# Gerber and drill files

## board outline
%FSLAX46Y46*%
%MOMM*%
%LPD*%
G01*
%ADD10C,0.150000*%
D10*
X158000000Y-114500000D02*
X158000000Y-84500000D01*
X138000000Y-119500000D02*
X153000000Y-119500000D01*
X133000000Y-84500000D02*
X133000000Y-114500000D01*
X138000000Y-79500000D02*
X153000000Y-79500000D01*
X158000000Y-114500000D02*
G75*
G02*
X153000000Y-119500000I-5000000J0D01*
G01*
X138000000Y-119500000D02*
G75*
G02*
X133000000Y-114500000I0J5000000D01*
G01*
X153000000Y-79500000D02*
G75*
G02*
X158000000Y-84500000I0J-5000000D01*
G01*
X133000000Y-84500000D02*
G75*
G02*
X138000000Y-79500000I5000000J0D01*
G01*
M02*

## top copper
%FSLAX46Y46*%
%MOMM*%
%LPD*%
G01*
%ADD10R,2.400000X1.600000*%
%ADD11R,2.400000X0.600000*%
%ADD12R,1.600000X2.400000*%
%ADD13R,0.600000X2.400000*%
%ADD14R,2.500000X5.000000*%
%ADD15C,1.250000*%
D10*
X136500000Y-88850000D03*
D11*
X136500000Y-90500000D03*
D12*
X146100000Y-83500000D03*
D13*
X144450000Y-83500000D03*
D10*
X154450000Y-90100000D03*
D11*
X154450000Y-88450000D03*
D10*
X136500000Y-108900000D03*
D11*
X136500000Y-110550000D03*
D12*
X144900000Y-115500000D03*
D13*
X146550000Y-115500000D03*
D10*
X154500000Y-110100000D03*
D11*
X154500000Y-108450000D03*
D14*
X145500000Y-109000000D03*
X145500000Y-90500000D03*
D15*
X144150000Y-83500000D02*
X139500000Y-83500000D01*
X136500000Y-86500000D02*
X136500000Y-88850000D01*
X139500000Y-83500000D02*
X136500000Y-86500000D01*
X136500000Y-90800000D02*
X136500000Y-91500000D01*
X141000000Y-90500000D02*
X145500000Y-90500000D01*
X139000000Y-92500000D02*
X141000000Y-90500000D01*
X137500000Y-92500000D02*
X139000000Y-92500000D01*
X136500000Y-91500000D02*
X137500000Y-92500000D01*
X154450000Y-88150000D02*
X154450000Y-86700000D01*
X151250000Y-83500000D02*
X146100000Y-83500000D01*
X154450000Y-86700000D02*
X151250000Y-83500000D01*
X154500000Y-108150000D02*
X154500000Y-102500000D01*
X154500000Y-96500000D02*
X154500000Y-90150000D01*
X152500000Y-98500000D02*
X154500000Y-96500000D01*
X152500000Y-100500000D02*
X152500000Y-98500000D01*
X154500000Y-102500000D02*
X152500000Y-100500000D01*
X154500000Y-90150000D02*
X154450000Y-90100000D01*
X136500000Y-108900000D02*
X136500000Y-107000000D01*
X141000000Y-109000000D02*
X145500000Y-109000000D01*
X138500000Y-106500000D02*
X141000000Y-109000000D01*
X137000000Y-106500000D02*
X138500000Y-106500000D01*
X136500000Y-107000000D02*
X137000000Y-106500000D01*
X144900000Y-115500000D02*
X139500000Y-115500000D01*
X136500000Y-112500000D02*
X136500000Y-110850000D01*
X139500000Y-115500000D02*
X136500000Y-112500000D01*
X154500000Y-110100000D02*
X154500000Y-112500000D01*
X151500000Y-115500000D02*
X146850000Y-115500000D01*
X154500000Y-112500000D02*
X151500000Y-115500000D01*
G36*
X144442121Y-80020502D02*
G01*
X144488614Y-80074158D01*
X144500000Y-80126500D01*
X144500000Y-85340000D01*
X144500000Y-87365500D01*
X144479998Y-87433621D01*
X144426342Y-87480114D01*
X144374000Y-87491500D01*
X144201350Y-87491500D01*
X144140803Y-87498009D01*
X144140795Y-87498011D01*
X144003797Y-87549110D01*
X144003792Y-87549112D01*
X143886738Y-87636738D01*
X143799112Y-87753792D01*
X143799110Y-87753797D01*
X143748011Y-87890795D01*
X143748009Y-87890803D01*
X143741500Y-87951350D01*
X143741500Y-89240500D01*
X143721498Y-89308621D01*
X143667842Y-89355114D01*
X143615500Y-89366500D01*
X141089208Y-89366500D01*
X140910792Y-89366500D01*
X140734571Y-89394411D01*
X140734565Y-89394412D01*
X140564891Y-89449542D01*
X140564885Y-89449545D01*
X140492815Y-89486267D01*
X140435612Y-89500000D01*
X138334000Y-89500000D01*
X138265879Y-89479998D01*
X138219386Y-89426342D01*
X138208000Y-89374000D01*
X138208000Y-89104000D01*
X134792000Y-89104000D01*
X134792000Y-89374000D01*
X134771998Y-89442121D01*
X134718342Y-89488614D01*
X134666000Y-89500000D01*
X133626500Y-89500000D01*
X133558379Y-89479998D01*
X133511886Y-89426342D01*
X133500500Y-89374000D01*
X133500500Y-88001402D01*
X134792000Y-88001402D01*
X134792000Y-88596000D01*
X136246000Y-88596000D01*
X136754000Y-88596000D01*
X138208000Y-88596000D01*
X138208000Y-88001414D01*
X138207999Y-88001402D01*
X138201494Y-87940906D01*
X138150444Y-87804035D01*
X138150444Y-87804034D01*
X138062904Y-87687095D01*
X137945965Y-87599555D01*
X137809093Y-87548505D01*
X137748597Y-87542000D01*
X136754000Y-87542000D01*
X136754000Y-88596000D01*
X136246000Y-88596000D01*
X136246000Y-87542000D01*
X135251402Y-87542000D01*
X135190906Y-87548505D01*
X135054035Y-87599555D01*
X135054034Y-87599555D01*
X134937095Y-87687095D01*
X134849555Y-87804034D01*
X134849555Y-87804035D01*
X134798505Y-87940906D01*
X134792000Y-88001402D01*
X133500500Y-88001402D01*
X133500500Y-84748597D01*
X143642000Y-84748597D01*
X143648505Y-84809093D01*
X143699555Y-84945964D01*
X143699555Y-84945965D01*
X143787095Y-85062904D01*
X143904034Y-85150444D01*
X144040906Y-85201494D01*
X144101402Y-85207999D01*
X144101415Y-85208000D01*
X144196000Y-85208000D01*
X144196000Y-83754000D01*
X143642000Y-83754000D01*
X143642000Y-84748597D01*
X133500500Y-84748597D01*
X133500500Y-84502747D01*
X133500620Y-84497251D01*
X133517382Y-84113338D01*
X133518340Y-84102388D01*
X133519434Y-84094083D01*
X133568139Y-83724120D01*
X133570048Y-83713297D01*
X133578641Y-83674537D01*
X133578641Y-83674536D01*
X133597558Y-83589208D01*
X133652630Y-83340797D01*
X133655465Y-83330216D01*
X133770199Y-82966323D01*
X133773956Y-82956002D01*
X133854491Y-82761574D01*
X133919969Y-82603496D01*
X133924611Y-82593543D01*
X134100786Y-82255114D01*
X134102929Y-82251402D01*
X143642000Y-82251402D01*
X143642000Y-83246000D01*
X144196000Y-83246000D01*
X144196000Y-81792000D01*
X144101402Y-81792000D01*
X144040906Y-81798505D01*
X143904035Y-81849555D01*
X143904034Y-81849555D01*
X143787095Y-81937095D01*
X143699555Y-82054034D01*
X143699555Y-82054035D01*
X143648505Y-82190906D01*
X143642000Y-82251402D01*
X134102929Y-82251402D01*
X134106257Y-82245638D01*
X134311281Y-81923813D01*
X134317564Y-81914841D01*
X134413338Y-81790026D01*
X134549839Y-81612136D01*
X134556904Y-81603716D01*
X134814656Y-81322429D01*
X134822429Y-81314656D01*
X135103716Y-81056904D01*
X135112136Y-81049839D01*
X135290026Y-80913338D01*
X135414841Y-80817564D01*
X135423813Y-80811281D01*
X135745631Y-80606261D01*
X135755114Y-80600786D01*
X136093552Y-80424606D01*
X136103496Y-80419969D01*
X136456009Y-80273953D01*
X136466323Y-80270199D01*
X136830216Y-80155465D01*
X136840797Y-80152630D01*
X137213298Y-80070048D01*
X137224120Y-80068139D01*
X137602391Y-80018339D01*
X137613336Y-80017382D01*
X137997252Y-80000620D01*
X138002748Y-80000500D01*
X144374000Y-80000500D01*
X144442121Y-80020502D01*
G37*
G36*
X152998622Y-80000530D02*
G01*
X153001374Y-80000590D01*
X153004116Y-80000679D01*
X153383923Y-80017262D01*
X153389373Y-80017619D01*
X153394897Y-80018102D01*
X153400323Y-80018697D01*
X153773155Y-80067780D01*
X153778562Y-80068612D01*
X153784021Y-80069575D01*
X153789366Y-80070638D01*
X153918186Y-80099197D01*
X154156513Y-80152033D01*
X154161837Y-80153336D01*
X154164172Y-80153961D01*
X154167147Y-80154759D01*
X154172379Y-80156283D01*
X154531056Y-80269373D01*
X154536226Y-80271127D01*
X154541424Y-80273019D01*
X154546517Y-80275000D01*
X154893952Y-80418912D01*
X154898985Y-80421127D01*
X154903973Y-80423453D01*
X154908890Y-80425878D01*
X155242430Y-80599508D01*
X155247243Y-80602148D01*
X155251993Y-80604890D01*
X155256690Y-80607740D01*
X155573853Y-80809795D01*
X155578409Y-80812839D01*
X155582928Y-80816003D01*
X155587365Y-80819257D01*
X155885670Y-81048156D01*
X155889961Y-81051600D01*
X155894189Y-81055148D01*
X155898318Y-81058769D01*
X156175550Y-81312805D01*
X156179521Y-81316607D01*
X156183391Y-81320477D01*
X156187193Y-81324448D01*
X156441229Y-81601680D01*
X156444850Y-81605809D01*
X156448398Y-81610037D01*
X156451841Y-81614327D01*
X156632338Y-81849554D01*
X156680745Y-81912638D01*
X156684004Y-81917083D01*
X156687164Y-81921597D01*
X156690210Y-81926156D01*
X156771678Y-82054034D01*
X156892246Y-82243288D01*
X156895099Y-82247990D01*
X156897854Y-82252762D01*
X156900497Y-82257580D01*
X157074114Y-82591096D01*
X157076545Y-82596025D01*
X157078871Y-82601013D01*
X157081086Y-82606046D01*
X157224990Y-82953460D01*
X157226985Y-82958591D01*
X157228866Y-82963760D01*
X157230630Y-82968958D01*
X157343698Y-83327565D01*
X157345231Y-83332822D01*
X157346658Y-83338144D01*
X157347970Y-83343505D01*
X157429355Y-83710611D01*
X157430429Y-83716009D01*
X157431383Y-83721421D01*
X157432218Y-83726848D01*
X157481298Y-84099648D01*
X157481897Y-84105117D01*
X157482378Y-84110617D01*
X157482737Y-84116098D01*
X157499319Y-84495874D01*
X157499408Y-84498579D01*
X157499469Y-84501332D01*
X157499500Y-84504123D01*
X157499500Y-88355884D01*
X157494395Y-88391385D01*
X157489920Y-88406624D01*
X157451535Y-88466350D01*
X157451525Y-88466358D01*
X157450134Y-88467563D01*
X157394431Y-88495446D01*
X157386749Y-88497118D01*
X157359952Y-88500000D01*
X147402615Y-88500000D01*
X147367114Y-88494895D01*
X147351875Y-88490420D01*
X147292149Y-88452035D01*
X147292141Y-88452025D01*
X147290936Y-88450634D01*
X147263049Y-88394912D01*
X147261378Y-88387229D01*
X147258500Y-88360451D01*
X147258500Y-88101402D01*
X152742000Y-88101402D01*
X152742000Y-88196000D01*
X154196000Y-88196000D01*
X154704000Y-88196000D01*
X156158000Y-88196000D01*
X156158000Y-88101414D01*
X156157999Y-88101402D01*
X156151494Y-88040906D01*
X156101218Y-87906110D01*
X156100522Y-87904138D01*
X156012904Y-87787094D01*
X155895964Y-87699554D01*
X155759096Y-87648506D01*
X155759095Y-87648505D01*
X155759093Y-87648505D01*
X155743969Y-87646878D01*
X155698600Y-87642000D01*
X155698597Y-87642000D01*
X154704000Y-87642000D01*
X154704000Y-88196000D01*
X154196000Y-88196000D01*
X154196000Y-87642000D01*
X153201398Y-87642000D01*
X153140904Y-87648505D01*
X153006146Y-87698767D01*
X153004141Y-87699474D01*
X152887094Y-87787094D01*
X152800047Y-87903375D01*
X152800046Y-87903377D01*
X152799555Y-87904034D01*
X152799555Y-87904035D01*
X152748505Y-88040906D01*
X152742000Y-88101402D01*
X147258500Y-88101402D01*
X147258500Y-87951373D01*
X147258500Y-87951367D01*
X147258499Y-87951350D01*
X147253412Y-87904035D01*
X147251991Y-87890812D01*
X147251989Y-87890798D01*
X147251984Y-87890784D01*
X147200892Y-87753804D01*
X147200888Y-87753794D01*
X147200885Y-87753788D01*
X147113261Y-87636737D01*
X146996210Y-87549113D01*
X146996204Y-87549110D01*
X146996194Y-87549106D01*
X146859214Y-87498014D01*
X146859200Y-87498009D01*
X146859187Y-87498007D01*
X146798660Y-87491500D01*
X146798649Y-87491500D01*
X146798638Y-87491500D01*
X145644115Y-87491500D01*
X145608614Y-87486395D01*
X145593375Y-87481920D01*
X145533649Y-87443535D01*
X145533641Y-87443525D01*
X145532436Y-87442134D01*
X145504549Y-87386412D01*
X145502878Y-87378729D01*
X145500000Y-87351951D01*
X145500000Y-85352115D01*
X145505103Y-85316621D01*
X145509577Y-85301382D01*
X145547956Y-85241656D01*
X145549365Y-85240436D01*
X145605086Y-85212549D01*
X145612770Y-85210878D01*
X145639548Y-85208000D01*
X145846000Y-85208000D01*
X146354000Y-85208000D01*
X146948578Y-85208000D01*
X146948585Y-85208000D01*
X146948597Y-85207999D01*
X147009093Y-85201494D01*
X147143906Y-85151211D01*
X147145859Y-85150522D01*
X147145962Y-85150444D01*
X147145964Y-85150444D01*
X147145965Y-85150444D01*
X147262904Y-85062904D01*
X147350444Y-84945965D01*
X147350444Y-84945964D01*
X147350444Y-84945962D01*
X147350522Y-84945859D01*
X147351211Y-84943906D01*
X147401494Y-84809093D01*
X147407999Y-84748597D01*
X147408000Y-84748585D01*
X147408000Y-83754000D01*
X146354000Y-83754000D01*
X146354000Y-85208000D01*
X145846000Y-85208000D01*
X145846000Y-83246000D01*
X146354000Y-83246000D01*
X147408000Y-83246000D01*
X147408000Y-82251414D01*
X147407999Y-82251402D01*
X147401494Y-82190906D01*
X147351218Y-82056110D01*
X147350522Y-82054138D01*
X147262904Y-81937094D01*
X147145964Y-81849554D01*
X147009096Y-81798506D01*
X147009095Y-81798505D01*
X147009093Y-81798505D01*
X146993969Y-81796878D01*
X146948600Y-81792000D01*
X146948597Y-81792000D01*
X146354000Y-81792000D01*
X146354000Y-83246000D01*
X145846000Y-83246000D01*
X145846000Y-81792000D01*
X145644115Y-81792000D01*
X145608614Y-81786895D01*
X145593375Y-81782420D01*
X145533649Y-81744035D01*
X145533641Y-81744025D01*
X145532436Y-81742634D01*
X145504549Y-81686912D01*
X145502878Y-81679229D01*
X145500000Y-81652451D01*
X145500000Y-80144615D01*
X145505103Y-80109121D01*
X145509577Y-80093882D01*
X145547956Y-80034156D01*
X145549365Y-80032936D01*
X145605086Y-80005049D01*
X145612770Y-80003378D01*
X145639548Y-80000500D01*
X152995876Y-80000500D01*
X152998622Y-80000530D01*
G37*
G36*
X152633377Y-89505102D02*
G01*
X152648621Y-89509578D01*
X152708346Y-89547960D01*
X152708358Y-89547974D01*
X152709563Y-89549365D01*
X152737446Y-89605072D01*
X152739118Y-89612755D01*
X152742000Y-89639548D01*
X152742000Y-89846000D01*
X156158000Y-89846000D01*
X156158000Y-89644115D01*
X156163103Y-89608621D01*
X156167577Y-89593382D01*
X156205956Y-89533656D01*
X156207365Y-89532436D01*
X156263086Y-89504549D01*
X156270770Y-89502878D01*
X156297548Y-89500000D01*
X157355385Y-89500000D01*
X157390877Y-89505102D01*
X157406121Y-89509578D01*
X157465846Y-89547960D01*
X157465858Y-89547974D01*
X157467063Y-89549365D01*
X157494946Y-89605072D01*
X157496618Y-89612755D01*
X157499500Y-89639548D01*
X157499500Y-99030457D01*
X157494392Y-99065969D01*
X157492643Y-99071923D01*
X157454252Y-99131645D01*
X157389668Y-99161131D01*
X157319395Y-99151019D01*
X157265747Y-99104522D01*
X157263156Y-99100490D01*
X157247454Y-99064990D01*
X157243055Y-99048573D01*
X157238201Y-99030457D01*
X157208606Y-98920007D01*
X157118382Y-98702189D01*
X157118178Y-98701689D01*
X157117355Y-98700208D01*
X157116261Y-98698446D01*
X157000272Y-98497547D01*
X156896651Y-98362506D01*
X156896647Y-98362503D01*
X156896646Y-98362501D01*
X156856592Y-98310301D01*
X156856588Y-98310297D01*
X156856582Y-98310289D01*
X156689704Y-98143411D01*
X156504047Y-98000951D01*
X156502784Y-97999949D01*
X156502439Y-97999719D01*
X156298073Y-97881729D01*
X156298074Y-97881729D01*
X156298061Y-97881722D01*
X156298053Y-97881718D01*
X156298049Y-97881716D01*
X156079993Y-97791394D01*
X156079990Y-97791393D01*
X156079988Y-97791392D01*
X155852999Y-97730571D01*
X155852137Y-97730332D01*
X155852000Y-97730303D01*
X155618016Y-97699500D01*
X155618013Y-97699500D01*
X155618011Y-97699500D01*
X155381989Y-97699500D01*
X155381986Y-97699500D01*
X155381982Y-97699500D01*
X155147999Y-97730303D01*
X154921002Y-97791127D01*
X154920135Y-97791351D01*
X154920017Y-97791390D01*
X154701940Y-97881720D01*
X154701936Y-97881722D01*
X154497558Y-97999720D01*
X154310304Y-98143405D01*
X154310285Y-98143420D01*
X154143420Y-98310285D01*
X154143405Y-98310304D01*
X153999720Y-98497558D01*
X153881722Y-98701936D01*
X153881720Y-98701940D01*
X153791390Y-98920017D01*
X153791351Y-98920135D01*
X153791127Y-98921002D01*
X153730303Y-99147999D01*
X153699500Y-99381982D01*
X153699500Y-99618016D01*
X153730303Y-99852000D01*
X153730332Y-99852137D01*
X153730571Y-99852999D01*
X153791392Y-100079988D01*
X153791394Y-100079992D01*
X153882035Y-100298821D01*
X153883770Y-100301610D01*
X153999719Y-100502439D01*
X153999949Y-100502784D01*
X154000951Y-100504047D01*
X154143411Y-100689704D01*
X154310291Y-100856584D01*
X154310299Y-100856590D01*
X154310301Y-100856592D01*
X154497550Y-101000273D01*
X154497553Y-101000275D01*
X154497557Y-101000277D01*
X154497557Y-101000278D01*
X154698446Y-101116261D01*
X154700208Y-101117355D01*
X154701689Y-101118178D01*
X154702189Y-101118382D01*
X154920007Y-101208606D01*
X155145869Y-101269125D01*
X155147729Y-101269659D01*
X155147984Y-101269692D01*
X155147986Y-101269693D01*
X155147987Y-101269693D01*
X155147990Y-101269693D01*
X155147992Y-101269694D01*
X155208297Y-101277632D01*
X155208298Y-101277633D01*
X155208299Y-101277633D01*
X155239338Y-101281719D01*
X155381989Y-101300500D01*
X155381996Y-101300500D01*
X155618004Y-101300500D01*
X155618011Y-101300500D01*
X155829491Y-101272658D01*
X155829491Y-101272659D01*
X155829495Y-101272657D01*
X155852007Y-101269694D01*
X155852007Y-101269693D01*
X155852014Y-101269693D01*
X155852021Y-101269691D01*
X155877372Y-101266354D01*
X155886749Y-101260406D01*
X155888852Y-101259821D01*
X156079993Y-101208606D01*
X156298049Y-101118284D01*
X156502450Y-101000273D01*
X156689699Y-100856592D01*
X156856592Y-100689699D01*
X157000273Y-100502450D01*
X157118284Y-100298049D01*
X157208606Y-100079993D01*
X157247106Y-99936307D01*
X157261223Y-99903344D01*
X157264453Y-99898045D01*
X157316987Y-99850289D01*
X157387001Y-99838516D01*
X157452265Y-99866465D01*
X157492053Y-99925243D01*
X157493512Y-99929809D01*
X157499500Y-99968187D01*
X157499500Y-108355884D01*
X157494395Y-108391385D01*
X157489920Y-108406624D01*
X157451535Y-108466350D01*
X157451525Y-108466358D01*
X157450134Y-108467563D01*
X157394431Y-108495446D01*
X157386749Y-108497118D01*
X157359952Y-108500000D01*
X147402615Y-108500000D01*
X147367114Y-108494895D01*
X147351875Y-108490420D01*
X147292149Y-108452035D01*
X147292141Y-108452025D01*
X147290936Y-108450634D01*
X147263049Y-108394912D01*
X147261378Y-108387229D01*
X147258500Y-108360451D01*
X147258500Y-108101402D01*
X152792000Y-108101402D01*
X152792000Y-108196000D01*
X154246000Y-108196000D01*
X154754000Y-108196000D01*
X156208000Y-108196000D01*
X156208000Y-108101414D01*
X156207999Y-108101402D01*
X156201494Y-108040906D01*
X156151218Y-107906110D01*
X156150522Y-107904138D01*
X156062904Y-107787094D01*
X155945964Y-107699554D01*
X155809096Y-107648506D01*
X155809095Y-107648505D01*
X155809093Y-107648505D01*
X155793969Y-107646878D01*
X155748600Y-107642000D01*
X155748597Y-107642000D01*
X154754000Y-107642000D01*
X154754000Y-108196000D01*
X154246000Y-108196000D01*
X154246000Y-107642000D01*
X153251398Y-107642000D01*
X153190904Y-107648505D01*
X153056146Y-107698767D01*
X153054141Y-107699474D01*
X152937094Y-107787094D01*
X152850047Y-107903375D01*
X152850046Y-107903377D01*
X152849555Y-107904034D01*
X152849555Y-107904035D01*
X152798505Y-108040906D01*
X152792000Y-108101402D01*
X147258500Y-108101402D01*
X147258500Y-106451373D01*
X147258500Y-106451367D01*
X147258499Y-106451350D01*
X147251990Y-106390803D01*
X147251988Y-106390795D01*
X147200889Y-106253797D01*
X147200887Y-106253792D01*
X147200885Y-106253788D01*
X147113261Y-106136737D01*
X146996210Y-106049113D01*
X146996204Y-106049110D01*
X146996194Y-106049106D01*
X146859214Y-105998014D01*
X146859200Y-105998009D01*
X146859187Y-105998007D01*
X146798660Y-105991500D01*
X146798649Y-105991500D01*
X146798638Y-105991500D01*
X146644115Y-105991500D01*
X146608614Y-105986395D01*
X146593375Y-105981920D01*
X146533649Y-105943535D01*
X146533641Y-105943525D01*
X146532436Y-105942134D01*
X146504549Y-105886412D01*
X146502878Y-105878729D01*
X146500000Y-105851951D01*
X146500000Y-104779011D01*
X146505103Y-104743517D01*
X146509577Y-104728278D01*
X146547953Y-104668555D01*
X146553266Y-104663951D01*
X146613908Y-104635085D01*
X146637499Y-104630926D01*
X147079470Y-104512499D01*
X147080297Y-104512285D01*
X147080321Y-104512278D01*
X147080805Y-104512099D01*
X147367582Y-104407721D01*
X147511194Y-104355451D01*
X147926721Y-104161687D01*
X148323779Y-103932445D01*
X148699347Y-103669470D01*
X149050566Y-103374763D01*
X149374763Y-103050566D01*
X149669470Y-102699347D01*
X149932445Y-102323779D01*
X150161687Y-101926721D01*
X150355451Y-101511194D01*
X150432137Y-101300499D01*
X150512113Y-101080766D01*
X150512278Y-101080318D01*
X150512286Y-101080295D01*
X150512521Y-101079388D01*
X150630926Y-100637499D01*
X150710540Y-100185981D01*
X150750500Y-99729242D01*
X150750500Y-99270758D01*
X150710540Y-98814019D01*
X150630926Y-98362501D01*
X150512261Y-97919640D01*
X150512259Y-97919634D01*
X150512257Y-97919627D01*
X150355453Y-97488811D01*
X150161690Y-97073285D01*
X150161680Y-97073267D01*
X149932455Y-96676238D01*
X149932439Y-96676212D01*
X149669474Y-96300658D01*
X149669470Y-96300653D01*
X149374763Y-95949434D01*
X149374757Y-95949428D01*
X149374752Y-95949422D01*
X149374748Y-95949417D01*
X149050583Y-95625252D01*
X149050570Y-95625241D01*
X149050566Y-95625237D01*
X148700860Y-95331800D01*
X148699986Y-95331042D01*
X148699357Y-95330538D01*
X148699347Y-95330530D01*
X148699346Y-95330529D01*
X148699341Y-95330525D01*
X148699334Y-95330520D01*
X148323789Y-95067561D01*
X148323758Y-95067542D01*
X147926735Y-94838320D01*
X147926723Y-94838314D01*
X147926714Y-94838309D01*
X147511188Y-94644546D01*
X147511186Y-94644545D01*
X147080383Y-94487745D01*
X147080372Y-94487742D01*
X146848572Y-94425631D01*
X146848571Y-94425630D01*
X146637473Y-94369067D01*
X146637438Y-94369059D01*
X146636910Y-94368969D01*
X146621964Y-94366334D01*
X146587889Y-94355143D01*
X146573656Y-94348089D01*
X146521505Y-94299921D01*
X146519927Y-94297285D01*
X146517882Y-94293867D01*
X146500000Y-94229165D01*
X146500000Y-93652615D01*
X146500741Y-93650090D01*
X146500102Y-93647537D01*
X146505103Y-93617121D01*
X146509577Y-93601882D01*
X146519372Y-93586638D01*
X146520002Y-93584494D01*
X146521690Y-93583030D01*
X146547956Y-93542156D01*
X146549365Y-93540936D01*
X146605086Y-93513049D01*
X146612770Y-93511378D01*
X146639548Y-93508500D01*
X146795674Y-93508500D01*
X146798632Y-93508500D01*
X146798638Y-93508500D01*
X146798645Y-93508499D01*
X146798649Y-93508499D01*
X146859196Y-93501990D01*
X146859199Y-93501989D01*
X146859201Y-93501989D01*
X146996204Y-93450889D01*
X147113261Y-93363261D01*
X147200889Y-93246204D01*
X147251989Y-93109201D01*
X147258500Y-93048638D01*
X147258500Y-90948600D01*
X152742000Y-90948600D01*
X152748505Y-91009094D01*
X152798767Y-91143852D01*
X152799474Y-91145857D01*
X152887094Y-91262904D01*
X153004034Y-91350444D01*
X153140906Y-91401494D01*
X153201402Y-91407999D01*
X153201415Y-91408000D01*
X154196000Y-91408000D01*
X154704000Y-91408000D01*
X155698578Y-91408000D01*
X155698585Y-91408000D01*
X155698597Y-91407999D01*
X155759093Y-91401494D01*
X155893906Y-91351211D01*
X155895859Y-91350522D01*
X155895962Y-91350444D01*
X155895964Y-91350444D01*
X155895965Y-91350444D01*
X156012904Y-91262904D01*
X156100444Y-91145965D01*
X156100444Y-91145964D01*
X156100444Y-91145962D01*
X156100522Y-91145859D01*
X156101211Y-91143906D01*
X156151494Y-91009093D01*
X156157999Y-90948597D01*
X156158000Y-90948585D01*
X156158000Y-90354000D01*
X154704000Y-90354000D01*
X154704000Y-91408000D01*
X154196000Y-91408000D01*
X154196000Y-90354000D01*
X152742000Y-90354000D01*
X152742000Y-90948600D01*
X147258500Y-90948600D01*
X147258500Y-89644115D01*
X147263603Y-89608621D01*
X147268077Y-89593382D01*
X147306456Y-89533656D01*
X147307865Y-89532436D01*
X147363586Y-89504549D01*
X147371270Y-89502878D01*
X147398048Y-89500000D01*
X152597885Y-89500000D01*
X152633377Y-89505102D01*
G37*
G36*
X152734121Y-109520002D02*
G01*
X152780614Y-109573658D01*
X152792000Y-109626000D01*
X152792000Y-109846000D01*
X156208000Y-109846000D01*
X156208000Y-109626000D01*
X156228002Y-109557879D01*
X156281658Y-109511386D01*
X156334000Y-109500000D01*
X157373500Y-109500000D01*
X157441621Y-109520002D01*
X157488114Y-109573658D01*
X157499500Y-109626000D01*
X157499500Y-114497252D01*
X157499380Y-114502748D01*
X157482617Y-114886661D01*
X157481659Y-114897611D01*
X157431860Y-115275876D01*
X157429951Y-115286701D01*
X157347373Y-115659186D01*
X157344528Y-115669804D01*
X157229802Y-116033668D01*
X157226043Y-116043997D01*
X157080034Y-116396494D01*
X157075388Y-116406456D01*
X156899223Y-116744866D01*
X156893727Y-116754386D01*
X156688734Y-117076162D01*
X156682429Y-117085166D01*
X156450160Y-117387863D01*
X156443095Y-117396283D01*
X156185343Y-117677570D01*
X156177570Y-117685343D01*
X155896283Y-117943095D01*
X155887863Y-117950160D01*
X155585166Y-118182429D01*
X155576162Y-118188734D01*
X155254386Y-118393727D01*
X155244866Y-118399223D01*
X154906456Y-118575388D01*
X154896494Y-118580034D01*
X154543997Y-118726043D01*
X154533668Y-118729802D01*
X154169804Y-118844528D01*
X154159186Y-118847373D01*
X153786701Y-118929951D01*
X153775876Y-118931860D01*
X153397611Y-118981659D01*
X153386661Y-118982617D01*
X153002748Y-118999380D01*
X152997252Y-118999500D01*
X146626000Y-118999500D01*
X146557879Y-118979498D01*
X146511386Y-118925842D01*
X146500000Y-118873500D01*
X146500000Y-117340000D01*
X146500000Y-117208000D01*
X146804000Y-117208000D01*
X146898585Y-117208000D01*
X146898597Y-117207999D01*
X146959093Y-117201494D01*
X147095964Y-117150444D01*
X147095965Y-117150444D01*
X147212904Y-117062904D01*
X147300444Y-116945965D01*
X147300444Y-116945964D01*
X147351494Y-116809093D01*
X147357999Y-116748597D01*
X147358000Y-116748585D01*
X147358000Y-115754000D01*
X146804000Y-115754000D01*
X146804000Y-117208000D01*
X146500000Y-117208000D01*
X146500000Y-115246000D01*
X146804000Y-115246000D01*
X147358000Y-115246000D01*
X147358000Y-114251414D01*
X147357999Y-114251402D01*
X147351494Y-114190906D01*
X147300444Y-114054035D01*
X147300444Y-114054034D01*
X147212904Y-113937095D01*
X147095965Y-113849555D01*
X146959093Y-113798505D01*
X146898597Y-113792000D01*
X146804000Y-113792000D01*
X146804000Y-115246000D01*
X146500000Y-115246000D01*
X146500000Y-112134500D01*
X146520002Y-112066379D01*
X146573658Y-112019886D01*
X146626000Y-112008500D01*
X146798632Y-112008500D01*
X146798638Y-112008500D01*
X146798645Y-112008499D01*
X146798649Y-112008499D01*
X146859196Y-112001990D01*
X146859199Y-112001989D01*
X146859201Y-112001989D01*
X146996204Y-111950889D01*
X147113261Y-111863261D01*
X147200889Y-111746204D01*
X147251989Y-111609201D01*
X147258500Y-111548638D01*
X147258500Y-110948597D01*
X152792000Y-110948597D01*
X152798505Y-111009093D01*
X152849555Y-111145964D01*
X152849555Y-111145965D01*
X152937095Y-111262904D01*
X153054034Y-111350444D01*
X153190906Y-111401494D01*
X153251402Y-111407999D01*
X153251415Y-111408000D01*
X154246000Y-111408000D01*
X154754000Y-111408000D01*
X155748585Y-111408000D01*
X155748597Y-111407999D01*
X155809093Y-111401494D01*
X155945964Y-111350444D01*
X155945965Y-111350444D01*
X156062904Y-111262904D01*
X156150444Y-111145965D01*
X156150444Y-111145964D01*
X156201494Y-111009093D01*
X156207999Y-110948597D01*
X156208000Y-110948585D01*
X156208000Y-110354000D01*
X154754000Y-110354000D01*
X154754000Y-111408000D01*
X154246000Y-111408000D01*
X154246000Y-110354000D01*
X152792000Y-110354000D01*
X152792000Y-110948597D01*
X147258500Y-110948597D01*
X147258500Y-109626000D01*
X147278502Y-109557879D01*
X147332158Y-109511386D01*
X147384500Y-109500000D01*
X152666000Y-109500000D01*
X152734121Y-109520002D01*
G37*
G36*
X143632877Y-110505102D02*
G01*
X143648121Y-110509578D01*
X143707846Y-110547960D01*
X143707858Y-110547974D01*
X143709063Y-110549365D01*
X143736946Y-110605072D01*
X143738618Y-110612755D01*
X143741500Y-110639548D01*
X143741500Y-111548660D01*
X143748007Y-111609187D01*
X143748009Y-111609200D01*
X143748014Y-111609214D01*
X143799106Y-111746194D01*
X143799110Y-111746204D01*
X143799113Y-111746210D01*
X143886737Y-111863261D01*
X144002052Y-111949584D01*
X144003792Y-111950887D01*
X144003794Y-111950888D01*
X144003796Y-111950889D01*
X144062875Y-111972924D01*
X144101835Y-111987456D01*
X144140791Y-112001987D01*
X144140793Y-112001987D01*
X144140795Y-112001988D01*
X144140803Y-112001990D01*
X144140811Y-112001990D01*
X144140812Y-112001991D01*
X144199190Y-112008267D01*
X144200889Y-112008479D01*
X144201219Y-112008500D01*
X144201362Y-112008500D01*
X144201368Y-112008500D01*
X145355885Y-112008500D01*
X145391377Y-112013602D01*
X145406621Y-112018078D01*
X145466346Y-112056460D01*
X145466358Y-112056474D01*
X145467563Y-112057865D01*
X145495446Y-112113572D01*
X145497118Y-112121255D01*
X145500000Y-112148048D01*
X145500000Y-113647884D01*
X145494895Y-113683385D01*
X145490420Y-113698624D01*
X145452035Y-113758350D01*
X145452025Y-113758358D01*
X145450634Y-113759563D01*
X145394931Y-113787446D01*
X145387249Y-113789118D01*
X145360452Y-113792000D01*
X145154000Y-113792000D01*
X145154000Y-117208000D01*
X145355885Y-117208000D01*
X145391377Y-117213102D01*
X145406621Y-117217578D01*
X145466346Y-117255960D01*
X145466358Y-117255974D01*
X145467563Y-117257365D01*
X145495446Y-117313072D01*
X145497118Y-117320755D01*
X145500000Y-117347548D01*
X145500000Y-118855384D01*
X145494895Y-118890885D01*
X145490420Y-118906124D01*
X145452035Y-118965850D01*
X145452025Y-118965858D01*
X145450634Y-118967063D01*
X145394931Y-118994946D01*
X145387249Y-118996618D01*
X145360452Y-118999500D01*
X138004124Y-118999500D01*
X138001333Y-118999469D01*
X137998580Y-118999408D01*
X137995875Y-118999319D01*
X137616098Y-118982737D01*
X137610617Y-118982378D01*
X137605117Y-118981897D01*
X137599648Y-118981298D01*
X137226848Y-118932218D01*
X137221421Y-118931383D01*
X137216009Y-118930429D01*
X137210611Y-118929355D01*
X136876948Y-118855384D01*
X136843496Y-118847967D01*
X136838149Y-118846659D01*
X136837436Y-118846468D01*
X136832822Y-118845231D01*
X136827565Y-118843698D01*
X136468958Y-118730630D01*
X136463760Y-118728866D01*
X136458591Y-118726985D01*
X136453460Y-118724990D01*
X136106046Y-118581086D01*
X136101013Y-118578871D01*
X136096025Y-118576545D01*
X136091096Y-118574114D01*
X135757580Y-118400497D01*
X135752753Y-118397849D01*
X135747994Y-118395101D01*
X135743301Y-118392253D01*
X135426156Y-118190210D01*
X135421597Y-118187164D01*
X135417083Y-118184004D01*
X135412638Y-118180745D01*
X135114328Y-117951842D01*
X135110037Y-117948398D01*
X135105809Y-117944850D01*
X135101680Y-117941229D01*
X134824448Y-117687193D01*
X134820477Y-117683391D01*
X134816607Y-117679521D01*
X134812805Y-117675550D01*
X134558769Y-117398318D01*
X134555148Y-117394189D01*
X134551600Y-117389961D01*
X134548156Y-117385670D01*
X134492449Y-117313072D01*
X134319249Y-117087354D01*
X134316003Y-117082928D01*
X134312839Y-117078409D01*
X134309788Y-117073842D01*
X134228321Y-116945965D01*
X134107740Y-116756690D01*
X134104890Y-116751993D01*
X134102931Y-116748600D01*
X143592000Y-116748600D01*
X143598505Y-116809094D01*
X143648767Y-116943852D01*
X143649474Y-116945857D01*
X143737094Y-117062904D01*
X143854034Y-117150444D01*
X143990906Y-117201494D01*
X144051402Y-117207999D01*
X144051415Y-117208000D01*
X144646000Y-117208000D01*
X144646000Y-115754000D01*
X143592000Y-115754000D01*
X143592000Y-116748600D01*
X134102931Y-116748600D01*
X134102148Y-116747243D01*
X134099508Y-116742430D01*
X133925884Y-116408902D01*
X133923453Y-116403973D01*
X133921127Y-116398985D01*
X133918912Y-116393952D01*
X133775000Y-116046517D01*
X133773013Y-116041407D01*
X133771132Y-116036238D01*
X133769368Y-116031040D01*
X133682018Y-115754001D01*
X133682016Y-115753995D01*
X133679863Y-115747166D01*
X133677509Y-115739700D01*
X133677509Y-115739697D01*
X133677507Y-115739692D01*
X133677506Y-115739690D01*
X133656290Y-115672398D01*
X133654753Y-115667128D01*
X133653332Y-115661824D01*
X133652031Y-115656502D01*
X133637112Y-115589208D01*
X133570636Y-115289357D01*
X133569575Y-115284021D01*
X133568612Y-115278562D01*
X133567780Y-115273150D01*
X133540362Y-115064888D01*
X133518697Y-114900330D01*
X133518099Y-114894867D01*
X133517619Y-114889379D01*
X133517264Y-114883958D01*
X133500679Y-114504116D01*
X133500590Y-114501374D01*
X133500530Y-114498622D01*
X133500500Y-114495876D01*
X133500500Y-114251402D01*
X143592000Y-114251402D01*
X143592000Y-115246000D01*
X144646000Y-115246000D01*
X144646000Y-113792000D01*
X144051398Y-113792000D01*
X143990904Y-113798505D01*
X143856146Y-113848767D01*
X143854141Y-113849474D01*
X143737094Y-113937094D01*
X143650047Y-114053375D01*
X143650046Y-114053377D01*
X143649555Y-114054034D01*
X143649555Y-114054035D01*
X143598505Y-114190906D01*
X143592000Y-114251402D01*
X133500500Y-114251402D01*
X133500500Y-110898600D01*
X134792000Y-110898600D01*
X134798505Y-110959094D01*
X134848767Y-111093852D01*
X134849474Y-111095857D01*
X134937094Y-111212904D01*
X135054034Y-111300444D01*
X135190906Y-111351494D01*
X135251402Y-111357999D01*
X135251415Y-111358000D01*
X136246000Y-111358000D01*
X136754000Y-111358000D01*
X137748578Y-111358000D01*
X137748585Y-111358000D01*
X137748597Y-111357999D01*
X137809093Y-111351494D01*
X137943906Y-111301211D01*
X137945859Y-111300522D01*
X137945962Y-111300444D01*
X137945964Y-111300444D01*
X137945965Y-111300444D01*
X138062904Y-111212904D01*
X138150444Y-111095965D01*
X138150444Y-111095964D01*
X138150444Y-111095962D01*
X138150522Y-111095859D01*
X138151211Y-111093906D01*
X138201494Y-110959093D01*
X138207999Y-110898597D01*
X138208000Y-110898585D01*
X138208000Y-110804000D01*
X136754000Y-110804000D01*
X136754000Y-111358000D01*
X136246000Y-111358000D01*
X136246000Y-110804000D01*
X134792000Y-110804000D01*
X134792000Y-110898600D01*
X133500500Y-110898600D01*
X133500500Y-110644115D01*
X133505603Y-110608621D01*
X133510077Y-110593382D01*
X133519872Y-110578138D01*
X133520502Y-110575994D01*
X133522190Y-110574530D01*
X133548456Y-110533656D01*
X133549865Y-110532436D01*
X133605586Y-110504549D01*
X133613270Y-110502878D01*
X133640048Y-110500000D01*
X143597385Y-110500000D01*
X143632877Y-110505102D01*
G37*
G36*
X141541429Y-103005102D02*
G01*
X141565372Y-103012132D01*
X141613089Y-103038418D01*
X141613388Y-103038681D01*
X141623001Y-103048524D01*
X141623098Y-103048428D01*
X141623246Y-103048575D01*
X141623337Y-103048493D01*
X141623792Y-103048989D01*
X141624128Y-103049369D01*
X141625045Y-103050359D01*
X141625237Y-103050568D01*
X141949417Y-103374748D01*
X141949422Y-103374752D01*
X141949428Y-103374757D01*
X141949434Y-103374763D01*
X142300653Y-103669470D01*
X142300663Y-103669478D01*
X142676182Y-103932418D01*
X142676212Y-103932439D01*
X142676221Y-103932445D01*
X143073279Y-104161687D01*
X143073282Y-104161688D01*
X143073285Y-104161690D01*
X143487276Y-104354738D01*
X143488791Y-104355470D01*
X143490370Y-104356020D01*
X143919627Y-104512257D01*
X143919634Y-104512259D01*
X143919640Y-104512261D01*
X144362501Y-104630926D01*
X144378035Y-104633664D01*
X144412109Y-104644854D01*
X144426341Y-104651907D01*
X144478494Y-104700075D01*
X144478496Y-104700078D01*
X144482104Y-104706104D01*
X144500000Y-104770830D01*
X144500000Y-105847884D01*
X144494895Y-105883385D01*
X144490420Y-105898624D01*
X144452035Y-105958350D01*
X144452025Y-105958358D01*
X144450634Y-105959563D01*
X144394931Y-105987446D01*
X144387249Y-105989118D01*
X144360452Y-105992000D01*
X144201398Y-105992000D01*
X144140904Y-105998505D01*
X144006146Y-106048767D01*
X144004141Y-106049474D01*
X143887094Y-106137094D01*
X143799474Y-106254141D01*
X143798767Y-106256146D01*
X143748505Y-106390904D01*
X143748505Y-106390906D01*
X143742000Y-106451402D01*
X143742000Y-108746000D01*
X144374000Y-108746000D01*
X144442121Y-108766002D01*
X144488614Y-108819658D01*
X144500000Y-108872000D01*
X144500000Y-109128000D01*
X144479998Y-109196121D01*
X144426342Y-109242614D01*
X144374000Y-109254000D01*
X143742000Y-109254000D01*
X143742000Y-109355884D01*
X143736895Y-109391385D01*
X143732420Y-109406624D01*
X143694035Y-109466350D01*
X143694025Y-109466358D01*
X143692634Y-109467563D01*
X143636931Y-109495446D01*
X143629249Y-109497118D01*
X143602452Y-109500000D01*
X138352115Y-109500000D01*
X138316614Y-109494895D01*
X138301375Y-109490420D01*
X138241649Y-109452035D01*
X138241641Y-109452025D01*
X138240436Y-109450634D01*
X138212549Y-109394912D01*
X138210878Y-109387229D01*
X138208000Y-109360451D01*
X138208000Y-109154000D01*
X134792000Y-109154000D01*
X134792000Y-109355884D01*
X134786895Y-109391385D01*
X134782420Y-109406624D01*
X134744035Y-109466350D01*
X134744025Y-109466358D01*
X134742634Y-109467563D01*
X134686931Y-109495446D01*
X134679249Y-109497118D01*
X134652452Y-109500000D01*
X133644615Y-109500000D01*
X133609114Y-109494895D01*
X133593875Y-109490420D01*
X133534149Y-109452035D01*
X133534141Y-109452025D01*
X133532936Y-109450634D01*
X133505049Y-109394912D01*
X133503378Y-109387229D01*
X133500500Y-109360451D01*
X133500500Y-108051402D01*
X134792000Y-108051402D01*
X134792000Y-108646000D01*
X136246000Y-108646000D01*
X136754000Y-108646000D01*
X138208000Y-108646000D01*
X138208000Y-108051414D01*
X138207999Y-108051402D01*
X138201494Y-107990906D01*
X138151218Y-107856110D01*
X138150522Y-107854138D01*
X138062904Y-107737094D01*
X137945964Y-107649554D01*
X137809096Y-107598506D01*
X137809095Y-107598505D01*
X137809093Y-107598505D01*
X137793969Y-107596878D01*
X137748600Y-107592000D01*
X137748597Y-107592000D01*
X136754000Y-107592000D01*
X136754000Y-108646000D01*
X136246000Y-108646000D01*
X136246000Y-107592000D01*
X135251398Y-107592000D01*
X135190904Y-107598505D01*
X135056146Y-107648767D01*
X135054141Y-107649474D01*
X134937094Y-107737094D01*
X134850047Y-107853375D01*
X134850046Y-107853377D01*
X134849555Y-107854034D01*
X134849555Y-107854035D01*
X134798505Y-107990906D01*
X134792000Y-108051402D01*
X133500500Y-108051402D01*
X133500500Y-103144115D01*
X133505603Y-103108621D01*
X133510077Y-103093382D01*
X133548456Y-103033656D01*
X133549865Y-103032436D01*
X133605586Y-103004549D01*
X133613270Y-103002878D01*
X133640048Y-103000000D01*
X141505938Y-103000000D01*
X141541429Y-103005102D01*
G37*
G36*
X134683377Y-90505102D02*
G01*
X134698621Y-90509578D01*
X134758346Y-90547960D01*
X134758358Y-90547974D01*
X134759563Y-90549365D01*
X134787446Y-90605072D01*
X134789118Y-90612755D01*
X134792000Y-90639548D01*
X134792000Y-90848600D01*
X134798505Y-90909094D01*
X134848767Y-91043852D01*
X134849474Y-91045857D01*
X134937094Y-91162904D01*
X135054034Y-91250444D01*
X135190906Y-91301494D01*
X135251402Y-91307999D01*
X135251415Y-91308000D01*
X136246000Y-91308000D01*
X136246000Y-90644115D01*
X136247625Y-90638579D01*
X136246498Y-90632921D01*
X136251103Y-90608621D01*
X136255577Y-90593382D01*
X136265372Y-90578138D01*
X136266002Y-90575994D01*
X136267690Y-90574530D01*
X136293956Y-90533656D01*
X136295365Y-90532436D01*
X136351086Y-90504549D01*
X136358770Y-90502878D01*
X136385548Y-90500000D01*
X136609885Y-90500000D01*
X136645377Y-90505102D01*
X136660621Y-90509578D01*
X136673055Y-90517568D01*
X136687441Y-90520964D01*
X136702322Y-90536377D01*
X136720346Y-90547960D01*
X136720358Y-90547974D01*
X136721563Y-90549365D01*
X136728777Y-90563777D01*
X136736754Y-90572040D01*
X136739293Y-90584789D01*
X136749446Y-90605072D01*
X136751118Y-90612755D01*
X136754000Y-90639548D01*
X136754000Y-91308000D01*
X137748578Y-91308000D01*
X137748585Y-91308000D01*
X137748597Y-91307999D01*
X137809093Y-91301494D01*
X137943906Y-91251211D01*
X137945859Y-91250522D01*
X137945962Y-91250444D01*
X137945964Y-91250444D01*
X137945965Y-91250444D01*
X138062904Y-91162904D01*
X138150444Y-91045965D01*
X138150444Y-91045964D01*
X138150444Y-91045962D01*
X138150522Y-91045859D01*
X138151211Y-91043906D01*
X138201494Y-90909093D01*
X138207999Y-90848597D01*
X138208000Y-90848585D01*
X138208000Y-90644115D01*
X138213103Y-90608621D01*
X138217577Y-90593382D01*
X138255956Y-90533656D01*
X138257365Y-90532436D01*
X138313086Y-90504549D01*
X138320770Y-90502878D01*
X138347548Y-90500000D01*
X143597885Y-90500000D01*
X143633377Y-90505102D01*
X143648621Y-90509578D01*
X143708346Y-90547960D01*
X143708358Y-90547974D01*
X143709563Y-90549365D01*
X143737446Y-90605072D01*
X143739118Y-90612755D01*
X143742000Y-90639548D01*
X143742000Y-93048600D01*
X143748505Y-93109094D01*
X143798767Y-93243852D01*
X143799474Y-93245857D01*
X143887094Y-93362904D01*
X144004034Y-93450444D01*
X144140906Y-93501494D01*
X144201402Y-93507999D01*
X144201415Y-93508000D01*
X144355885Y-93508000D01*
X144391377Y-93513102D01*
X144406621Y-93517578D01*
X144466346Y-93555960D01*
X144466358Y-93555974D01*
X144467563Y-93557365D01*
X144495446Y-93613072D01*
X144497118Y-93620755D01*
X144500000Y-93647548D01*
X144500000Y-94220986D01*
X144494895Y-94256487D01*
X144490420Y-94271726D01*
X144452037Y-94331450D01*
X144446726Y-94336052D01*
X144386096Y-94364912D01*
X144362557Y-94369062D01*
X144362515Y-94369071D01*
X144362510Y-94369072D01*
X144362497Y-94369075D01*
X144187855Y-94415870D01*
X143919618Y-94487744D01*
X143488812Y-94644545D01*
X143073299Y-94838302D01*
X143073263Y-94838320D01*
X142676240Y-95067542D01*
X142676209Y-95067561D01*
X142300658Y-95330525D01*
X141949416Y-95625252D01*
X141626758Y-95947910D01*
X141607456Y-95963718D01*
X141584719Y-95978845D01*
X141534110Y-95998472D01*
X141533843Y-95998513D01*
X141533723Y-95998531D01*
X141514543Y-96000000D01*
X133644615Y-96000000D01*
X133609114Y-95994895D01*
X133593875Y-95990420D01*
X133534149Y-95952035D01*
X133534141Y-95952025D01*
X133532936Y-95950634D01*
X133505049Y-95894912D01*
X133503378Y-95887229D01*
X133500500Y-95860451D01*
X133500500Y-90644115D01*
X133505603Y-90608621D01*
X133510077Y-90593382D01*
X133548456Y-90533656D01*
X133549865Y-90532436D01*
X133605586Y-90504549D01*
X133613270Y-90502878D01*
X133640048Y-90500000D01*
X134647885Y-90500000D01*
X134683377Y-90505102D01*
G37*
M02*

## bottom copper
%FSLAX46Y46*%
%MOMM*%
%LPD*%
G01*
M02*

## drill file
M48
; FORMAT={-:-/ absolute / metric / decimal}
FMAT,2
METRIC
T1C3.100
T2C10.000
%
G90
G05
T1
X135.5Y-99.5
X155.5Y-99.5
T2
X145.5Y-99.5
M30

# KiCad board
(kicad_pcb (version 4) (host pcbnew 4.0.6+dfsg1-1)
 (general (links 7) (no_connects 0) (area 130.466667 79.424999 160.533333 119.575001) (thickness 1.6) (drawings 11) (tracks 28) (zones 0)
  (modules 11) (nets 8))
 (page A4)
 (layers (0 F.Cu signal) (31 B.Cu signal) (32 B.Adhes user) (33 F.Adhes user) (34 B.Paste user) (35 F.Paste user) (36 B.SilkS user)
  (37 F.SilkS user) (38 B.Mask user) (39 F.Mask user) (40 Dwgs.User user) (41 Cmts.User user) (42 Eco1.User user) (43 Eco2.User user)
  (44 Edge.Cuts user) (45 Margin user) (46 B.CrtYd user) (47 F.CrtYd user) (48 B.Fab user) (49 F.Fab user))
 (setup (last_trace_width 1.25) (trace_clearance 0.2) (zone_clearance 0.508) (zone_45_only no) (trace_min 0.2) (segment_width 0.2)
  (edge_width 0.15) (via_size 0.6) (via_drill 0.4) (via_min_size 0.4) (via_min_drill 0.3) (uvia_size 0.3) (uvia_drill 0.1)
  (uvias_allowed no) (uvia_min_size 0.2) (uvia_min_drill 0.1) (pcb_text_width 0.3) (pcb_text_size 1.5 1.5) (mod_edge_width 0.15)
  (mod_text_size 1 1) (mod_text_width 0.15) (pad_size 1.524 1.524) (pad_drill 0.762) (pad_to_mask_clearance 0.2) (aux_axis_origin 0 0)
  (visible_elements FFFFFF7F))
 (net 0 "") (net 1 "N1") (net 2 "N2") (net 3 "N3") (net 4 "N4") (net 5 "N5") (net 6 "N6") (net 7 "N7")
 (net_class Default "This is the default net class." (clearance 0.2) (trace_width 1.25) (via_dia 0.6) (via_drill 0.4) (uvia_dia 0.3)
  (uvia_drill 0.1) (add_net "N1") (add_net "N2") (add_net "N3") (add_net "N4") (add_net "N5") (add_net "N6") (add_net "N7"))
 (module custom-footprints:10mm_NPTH (layer F.Cu) (at 145.5 99.5)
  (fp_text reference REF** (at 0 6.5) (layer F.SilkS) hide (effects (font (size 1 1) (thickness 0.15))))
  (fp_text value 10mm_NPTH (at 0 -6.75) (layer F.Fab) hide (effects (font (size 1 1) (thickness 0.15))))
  (pad "" np_thru_hole circle (at 0 0) (size 10 10) (drill 10) (layers *.Cu *.Mask)))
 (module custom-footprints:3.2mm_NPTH (layer F.Cu) (at 135.5 99.5)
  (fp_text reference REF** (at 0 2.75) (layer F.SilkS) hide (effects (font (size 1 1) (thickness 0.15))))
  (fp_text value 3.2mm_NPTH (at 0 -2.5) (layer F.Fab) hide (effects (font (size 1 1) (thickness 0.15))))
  (pad "" np_thru_hole circle (at 0 0) (size 3.1 3.1) (drill 3.1) (layers *.Cu *.Mask)))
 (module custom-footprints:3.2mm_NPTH (layer F.Cu) (at 155.5 99.5)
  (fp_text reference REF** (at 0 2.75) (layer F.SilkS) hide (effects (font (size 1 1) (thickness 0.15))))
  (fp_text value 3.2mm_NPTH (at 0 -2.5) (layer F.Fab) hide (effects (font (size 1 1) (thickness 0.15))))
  (pad "" np_thru_hole circle (at 0 0) (size 3.1 3.1) (drill 3.1) (layers *.Cu *.Mask)))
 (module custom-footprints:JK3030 (layer F.Cu) (at 136.5 89.45 270)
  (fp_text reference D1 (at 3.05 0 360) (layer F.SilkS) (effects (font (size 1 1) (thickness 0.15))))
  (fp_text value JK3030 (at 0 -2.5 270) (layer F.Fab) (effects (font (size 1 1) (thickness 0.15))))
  (pad 1 smd rect (at -0.6 0 270) (size 1.6 2.4) (layers F.Cu F.Paste F.Mask) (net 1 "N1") (solder_paste_margin -0.15))
  (pad 2 smd rect (at 1.35 0 270) (size 0.6 2.4) (drill (offset -0.3 0)) (layers F.Cu F.Paste F.Mask) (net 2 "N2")
   (solder_paste_margin -0.1)))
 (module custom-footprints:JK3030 (layer F.Cu) (at 145.5 83.5 180)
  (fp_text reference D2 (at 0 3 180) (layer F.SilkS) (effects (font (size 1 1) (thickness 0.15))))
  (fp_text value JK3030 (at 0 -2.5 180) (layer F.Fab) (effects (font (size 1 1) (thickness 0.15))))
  (pad 1 smd rect (at -0.6 0 180) (size 1.6 2.4) (layers F.Cu F.Paste F.Mask) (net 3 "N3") (solder_paste_margin -0.15))
  (pad 2 smd rect (at 1.35 0 180) (size 0.6 2.4) (drill (offset -0.3 0)) (layers F.Cu F.Paste F.Mask) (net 1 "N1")
   (solder_paste_margin -0.1)))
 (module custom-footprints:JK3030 (layer F.Cu) (at 154.45 89.5 90)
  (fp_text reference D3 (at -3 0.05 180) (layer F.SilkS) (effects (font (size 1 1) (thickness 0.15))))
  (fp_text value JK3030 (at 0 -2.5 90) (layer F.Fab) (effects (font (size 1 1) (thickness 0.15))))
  (pad 1 smd rect (at -0.6 0 90) (size 1.6 2.4) (layers F.Cu F.Paste F.Mask) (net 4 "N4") (solder_paste_margin -0.15))
  (pad 2 smd rect (at 1.35 0 90) (size 0.6 2.4) (drill (offset -0.3 0)) (layers F.Cu F.Paste F.Mask) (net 3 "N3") (solder_paste_margin -0.1)))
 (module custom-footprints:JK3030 (layer F.Cu) (at 136.5 109.5 270)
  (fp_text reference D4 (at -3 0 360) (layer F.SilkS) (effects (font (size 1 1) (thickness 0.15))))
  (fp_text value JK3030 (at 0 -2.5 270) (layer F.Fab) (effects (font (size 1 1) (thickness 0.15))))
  (pad 1 smd rect (at -0.6 0 270) (size 1.6 2.4) (layers F.Cu F.Paste F.Mask) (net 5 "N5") (solder_paste_margin -0.15))
  (pad 2 smd rect (at 1.35 0 270) (size 0.6 2.4) (drill (offset -0.3 0)) (layers F.Cu F.Paste F.Mask) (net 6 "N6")
   (solder_paste_margin -0.1)))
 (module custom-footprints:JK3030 (layer F.Cu) (at 145.5 115.5)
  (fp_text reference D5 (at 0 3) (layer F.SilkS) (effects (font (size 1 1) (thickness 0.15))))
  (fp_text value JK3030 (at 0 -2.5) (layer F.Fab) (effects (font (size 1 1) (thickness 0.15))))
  (pad 1 smd rect (at -0.6 0) (size 1.6 2.4) (layers F.Cu F.Paste F.Mask) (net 6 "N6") (solder_paste_margin -0.15))
  (pad 2 smd rect (at 1.35 0) (size 0.6 2.4) (drill (offset -0.3 0)) (layers F.Cu F.Paste F.Mask) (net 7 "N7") (solder_paste_margin -0.1)))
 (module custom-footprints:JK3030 (layer F.Cu) (at 154.5 109.5 90)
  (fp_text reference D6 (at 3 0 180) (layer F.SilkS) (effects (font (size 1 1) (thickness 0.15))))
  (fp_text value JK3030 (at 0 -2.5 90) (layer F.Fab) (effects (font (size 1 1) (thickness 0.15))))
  (pad 1 smd rect (at -0.6 0 90) (size 1.6 2.4) (layers F.Cu F.Paste F.Mask) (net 7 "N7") (solder_paste_margin -0.15))
  (pad 2 smd rect (at 1.35 0 90) (size 0.6 2.4) (drill (offset -0.3 0)) (layers F.Cu F.Paste F.Mask) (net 4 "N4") (solder_paste_margin -0.1)))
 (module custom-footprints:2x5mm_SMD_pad (layer F.Cu) (at 145.5 109)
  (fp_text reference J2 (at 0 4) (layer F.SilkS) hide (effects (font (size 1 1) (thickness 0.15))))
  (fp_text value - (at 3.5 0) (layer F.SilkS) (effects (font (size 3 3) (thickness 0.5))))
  (pad 1 smd rect (at 0 0) (size 2.5 5) (layers F.Cu F.Paste F.Mask) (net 5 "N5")))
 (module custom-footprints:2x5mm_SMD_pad (layer F.Cu) (at 145.5 90.5)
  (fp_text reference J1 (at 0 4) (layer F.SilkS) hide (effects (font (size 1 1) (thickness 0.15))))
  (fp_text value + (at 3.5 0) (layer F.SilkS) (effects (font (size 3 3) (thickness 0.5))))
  (pad 1 smd rect (at 0 0) (size 2.5 5) (layers F.Cu F.Paste F.Mask) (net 2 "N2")))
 (gr_line (start 158 114.5) (end 158 84.5) (angle 90) (layer Edge.Cuts) (width 0.15))
 (gr_line (start 138 119.5) (end 153 119.5) (angle 90) (layer Edge.Cuts) (width 0.15))
 (gr_line (start 133 84.5) (end 133 114.5) (angle 90) (layer Edge.Cuts) (width 0.15))
 (gr_line (start 138 79.5) (end 153 79.5) (angle 90) (layer Edge.Cuts) (width 0.15))
 (gr_arc (start 153 114.5) (end 158 114.5) (angle 90) (layer Edge.Cuts) (width 0.15))
 (gr_arc (start 138 114.5) (end 138 119.5) (angle 90) (layer Edge.Cuts) (width 0.15))
 (gr_arc (start 153 84.5) (end 153 79.5) (angle 90) (layer Edge.Cuts) (width 0.15))
 (gr_arc (start 138 84.5) (end 133 84.5) (angle 90) (layer Edge.Cuts) (width 0.15))
 (segment (start 144.15 83.5) (end 139.5 83.5) (width 1.25) (layer F.Cu) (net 1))
 (segment (start 136.5 86.5) (end 136.5 88.85) (width 1.25) (layer F.Cu) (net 1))
 (segment (start 139.5 83.5) (end 136.5 86.5) (width 1.25) (layer F.Cu) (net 1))
 (segment (start 136.5 90.8) (end 136.5 91.5) (width 1.25) (layer F.Cu) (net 2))
 (segment (start 141 90.5) (end 145.5 90.5) (width 1.25) (layer F.Cu) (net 2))
 (segment (start 139 92.5) (end 141 90.5) (width 1.25) (layer F.Cu) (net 2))
 (segment (start 137.5 92.5) (end 139 92.5) (width 1.25) (layer F.Cu) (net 2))
 (segment (start 136.5 91.5) (end 137.5 92.5) (width 1.25) (layer F.Cu) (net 2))
 (segment (start 154.45 88.15) (end 154.45 86.7) (width 1.25) (layer F.Cu) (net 3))
 (segment (start 151.25 83.5) (end 146.1 83.5) (width 1.25) (layer F.Cu) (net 3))
 (segment (start 154.45 86.7) (end 151.25 83.5) (width 1.25) (layer F.Cu) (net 3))
 (segment (start 154.5 108.15) (end 154.5 102.5) (width 1.25) (layer F.Cu) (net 4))
 (segment (start 154.5 96.5) (end 154.5 90.15) (width 1.25) (layer F.Cu) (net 4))
 (segment (start 152.5 98.5) (end 154.5 96.5) (width 1.25) (layer F.Cu) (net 4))
 (segment (start 152.5 100.5) (end 152.5 98.5) (width 1.25) (layer F.Cu) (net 4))
 (segment (start 154.5 102.5) (end 152.5 100.5) (width 1.25) (layer F.Cu) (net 4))
 (segment (start 154.5 90.15) (end 154.45 90.1) (width 1.25) (layer F.Cu) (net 4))
 (segment (start 136.5 108.9) (end 136.5 107) (width 1.25) (layer F.Cu) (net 5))
 (segment (start 141 109) (end 145.5 109) (width 1.25) (layer F.Cu) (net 5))
 (segment (start 138.5 106.5) (end 141 109) (width 1.25) (layer F.Cu) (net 5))
 (segment (start 137 106.5) (end 138.5 106.5) (width 1.25) (layer F.Cu) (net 5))
 (segment (start 136.5 107) (end 137 106.5) (width 1.25) (layer F.Cu) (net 5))
 (segment (start 144.9 115.5) (end 139.5 115.5) (width 1.25) (layer F.Cu) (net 6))
 (segment (start 136.5 112.5) (end 136.5 110.85) (width 1.25) (layer F.Cu) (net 6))
 (segment (start 139.5 115.5) (end 136.5 112.5) (width 1.25) (layer F.Cu) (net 6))
 (segment (start 154.5 110.1) (end 154.5 112.5) (width 1.25) (layer F.Cu) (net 7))
 (segment (start 151.5 115.5) (end 146.85 115.5) (width 1.25) (layer F.Cu) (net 7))
 (segment (start 154.5 112.5) (end 151.5 115.5) (width 1.25) (layer F.Cu) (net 7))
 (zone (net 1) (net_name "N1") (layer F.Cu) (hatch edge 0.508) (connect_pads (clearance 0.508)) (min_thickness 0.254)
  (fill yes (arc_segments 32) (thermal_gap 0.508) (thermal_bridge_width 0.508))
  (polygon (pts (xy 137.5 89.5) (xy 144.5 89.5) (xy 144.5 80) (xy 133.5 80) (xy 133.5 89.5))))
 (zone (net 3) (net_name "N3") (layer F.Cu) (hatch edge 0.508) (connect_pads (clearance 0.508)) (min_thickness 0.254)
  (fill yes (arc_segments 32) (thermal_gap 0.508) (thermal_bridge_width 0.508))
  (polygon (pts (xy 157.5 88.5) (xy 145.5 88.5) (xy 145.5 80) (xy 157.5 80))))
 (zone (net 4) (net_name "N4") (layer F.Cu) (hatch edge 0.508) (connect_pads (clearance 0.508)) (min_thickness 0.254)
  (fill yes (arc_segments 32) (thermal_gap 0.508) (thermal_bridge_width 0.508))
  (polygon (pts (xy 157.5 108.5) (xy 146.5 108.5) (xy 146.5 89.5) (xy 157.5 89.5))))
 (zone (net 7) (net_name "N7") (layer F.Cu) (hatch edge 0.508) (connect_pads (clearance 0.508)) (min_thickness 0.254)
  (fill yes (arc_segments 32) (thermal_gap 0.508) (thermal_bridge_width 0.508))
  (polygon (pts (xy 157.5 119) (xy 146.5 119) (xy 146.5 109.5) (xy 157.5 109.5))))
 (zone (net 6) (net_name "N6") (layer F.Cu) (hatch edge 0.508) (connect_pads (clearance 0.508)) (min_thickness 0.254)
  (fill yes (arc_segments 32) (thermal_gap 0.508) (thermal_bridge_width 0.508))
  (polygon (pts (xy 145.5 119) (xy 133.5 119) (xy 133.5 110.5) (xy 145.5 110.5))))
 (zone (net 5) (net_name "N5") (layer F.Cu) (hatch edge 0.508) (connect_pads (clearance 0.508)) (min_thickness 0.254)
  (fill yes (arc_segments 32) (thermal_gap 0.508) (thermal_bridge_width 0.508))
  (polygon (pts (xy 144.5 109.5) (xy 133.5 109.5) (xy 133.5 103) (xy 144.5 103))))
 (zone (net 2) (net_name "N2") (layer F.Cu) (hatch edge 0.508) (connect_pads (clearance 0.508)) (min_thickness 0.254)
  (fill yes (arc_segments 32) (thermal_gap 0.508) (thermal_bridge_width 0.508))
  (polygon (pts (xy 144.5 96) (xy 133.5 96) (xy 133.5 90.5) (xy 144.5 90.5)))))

